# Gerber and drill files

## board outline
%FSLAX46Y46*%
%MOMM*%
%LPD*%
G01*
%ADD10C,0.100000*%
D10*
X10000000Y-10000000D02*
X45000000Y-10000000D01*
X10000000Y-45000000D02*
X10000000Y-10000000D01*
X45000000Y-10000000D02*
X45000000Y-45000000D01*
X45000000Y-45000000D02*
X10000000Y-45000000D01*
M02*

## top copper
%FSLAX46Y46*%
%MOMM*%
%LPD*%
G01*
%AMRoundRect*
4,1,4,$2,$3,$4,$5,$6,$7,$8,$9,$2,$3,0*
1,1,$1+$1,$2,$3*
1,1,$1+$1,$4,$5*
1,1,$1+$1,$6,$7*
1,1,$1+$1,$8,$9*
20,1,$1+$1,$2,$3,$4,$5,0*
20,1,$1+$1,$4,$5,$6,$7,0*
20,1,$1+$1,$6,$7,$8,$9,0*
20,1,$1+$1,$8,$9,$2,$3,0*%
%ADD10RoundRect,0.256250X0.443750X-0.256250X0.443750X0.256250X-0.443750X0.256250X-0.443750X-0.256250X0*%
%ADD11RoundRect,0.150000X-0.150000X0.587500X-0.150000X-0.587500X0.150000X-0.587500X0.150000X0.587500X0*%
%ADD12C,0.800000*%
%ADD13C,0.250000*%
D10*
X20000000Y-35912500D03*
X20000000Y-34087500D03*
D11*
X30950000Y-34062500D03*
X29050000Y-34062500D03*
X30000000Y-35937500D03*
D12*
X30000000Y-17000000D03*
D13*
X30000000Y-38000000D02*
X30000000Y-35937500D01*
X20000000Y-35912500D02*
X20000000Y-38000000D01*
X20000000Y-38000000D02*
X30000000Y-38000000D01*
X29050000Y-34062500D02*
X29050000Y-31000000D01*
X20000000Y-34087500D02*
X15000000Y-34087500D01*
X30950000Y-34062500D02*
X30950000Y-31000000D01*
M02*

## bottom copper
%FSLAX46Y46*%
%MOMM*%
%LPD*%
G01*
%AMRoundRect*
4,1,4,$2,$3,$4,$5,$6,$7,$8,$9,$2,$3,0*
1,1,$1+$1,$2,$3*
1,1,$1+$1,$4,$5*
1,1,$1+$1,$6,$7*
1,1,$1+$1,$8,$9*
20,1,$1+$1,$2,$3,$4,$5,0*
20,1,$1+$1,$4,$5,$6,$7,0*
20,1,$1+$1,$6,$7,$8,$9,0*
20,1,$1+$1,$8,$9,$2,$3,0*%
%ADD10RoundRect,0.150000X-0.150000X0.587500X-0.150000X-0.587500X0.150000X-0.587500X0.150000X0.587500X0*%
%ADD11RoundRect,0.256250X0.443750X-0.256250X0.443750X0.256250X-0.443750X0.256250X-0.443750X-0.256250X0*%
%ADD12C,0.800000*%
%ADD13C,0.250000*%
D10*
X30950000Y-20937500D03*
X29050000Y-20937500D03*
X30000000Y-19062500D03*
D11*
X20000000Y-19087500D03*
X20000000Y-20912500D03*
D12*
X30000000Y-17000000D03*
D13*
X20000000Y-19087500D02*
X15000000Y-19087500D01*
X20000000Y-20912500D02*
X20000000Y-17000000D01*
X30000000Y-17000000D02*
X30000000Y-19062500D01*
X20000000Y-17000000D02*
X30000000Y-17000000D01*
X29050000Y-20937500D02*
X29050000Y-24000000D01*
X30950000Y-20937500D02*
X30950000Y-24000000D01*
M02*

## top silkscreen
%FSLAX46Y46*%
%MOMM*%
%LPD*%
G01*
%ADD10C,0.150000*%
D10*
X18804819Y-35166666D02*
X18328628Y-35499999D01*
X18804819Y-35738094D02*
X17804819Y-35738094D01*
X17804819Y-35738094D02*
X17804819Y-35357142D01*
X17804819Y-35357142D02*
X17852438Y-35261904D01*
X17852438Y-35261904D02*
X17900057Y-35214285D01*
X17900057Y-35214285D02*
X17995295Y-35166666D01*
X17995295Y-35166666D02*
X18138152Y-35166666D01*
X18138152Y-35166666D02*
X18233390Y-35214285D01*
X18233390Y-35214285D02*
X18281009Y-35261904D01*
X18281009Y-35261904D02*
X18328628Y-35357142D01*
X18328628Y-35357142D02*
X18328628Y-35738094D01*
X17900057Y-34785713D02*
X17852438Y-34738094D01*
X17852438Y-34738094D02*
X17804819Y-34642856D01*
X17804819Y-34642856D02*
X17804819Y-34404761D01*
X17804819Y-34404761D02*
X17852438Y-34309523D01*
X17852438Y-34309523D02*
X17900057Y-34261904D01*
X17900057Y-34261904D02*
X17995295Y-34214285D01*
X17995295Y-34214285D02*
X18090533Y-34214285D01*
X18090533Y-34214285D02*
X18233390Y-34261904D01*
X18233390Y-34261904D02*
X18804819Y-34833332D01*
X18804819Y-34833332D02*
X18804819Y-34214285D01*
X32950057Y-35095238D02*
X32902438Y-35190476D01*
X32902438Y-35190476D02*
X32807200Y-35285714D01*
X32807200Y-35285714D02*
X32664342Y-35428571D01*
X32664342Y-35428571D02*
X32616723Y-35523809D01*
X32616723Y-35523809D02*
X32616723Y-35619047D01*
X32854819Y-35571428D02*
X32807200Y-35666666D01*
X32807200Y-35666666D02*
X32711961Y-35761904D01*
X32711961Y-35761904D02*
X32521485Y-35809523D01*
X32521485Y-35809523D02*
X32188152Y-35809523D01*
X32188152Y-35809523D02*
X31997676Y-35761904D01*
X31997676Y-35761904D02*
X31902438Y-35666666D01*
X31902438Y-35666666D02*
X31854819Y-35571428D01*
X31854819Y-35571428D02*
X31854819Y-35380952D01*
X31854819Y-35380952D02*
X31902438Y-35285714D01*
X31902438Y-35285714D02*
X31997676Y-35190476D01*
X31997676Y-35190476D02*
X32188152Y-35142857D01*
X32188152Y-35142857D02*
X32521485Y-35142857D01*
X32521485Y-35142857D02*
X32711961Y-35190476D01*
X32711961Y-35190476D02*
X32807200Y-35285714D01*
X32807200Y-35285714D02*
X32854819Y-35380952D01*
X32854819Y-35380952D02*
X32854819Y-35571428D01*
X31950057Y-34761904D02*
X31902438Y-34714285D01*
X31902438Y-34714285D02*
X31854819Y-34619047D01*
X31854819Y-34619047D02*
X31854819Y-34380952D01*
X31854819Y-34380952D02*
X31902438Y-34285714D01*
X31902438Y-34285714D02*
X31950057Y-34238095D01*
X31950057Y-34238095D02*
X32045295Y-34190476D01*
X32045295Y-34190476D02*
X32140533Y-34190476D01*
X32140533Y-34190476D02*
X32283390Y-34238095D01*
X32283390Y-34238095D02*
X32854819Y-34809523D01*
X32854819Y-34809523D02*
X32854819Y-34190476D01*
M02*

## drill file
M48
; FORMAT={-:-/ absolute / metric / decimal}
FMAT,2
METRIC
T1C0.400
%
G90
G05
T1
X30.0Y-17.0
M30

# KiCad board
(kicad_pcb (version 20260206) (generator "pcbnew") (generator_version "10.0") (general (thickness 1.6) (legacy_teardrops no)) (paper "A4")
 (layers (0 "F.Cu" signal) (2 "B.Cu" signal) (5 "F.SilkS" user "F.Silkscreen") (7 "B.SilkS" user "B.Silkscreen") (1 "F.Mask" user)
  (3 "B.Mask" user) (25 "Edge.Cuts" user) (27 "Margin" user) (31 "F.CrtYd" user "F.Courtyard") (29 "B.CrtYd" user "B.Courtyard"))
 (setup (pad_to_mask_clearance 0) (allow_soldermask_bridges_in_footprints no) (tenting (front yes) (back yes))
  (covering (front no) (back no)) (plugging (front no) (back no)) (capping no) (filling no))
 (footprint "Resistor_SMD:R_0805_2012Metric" (layer "F.Cu") (at 20 35 90)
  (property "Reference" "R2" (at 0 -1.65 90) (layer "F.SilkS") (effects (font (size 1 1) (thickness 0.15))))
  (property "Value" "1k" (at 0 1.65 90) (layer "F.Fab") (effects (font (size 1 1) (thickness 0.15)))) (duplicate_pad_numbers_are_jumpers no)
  (pad "1" smd roundrect (at -0.9125 0 90) (size 1.025 1.4) (layers "F.Cu" "F.Mask" "F.Paste") (roundrect_rratio 0.25) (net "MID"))
  (pad "2" smd roundrect (at 0.9125 0 90) (size 1.025 1.4) (layers "F.Cu" "F.Mask" "F.Paste") (roundrect_rratio 0.25) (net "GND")))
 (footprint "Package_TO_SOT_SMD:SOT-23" (layer "F.Cu") (at 30 35 -90)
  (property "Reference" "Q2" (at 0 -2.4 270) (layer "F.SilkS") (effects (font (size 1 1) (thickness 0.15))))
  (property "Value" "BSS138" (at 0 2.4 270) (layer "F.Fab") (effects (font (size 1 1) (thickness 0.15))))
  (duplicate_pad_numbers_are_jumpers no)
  (pad "1" smd roundrect (at -0.9375 -0.95 270) (size 1.475 0.6) (layers "F.Cu" "F.Mask" "F.Paste") (roundrect_rratio 0.25) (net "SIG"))
  (pad "2" smd roundrect (at -0.9375 0.95 270) (size 1.475 0.6) (layers "F.Cu" "F.Mask" "F.Paste") (roundrect_rratio 0.25) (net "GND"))
  (pad "3" smd roundrect (at 0.9375 0 270) (size 1.475 0.6) (layers "F.Cu" "F.Mask" "F.Paste") (roundrect_rratio 0.25) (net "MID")))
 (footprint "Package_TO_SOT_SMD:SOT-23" (layer "B.Cu") (at 30 20 -90)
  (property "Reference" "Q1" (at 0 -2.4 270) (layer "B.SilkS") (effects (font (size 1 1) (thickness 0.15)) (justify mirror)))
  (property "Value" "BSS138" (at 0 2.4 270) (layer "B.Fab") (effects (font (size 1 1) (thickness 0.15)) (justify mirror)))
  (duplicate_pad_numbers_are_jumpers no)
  (pad "1" smd roundrect (at 0.9375 -0.95 270) (size 1.475 0.6) (layers "B.Cu" "B.Mask" "B.Paste") (roundrect_rratio 0.25) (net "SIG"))
  (pad "2" smd roundrect (at 0.9375 0.95 270) (size 1.475 0.6) (layers "B.Cu" "B.Mask" "B.Paste") (roundrect_rratio 0.25) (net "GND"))
  (pad "3" smd roundrect (at -0.9375 0 270) (size 1.475 0.6) (layers "B.Cu" "B.Mask" "B.Paste") (roundrect_rratio 0.25) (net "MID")))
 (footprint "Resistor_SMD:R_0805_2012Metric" (layer "B.Cu") (at 20 20 90)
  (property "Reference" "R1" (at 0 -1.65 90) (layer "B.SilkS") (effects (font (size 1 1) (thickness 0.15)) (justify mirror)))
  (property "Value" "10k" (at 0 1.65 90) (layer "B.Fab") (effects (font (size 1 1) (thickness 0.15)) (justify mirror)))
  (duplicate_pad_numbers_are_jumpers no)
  (pad "1" smd roundrect (at 0.9125 0 90) (size 1.025 1.4) (layers "B.Cu" "B.Mask" "B.Paste") (roundrect_rratio 0.25) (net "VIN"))
  (pad "2" smd roundrect (at -0.9125 0 90) (size 1.025 1.4) (layers "B.Cu" "B.Mask" "B.Paste") (roundrect_rratio 0.25) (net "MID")))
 (gr_line (start 10 10) (end 45 10) (stroke (width 0.1) (type default)) (layer "Edge.Cuts"))
 (gr_line (start 10 45) (end 10 10) (stroke (width 0.1) (type default)) (layer "Edge.Cuts"))
 (gr_line (start 45 10) (end 45 45) (stroke (width 0.1) (type default)) (layer "Edge.Cuts"))
 (gr_line (start 45 45) (end 10 45) (stroke (width 0.1) (type default)) (layer "Edge.Cuts"))
 (segment (start 20 19.0875) (end 15 19.0875) (width 0.25) (layer "B.Cu") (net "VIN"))
 (segment (start 30 38) (end 30 35.9375) (width 0.25) (layer "F.Cu") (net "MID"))
 (segment (start 20 35.9125) (end 20 38) (width 0.25) (layer "F.Cu") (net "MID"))
 (segment (start 20 38) (end 30 38) (width 0.25) (layer "F.Cu") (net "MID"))
 (via (at 30 17) (size 0.8) (drill 0.4) (layers "F.Cu" "B.Cu") (capping no) (covering (front no) (back no)) (plugging (front no) (back no))
  (filling no) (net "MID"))
 (segment (start 20 20.9125) (end 20 17) (width 0.25) (layer "B.Cu") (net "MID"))
 (segment (start 30 17) (end 30 19.0625) (width 0.25) (layer "B.Cu") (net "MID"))
 (segment (start 20 17) (end 30 17) (width 0.25) (layer "B.Cu") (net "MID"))
 (segment (start 29.05 34.0625) (end 29.05 31) (width 0.25) (layer "F.Cu") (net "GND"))
 (segment (start 20 34.0875) (end 15 34.0875) (width 0.25) (layer "F.Cu") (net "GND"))
 (segment (start 29.05 20.9375) (end 29.05 24) (width 0.25) (layer "B.Cu") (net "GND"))
 (segment (start 30.95 34.0625) (end 30.95 31) (width 0.25) (layer "F.Cu") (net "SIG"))
 (segment (start 30.95 20.9375) (end 30.95 24) (width 0.25) (layer "B.Cu") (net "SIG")))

